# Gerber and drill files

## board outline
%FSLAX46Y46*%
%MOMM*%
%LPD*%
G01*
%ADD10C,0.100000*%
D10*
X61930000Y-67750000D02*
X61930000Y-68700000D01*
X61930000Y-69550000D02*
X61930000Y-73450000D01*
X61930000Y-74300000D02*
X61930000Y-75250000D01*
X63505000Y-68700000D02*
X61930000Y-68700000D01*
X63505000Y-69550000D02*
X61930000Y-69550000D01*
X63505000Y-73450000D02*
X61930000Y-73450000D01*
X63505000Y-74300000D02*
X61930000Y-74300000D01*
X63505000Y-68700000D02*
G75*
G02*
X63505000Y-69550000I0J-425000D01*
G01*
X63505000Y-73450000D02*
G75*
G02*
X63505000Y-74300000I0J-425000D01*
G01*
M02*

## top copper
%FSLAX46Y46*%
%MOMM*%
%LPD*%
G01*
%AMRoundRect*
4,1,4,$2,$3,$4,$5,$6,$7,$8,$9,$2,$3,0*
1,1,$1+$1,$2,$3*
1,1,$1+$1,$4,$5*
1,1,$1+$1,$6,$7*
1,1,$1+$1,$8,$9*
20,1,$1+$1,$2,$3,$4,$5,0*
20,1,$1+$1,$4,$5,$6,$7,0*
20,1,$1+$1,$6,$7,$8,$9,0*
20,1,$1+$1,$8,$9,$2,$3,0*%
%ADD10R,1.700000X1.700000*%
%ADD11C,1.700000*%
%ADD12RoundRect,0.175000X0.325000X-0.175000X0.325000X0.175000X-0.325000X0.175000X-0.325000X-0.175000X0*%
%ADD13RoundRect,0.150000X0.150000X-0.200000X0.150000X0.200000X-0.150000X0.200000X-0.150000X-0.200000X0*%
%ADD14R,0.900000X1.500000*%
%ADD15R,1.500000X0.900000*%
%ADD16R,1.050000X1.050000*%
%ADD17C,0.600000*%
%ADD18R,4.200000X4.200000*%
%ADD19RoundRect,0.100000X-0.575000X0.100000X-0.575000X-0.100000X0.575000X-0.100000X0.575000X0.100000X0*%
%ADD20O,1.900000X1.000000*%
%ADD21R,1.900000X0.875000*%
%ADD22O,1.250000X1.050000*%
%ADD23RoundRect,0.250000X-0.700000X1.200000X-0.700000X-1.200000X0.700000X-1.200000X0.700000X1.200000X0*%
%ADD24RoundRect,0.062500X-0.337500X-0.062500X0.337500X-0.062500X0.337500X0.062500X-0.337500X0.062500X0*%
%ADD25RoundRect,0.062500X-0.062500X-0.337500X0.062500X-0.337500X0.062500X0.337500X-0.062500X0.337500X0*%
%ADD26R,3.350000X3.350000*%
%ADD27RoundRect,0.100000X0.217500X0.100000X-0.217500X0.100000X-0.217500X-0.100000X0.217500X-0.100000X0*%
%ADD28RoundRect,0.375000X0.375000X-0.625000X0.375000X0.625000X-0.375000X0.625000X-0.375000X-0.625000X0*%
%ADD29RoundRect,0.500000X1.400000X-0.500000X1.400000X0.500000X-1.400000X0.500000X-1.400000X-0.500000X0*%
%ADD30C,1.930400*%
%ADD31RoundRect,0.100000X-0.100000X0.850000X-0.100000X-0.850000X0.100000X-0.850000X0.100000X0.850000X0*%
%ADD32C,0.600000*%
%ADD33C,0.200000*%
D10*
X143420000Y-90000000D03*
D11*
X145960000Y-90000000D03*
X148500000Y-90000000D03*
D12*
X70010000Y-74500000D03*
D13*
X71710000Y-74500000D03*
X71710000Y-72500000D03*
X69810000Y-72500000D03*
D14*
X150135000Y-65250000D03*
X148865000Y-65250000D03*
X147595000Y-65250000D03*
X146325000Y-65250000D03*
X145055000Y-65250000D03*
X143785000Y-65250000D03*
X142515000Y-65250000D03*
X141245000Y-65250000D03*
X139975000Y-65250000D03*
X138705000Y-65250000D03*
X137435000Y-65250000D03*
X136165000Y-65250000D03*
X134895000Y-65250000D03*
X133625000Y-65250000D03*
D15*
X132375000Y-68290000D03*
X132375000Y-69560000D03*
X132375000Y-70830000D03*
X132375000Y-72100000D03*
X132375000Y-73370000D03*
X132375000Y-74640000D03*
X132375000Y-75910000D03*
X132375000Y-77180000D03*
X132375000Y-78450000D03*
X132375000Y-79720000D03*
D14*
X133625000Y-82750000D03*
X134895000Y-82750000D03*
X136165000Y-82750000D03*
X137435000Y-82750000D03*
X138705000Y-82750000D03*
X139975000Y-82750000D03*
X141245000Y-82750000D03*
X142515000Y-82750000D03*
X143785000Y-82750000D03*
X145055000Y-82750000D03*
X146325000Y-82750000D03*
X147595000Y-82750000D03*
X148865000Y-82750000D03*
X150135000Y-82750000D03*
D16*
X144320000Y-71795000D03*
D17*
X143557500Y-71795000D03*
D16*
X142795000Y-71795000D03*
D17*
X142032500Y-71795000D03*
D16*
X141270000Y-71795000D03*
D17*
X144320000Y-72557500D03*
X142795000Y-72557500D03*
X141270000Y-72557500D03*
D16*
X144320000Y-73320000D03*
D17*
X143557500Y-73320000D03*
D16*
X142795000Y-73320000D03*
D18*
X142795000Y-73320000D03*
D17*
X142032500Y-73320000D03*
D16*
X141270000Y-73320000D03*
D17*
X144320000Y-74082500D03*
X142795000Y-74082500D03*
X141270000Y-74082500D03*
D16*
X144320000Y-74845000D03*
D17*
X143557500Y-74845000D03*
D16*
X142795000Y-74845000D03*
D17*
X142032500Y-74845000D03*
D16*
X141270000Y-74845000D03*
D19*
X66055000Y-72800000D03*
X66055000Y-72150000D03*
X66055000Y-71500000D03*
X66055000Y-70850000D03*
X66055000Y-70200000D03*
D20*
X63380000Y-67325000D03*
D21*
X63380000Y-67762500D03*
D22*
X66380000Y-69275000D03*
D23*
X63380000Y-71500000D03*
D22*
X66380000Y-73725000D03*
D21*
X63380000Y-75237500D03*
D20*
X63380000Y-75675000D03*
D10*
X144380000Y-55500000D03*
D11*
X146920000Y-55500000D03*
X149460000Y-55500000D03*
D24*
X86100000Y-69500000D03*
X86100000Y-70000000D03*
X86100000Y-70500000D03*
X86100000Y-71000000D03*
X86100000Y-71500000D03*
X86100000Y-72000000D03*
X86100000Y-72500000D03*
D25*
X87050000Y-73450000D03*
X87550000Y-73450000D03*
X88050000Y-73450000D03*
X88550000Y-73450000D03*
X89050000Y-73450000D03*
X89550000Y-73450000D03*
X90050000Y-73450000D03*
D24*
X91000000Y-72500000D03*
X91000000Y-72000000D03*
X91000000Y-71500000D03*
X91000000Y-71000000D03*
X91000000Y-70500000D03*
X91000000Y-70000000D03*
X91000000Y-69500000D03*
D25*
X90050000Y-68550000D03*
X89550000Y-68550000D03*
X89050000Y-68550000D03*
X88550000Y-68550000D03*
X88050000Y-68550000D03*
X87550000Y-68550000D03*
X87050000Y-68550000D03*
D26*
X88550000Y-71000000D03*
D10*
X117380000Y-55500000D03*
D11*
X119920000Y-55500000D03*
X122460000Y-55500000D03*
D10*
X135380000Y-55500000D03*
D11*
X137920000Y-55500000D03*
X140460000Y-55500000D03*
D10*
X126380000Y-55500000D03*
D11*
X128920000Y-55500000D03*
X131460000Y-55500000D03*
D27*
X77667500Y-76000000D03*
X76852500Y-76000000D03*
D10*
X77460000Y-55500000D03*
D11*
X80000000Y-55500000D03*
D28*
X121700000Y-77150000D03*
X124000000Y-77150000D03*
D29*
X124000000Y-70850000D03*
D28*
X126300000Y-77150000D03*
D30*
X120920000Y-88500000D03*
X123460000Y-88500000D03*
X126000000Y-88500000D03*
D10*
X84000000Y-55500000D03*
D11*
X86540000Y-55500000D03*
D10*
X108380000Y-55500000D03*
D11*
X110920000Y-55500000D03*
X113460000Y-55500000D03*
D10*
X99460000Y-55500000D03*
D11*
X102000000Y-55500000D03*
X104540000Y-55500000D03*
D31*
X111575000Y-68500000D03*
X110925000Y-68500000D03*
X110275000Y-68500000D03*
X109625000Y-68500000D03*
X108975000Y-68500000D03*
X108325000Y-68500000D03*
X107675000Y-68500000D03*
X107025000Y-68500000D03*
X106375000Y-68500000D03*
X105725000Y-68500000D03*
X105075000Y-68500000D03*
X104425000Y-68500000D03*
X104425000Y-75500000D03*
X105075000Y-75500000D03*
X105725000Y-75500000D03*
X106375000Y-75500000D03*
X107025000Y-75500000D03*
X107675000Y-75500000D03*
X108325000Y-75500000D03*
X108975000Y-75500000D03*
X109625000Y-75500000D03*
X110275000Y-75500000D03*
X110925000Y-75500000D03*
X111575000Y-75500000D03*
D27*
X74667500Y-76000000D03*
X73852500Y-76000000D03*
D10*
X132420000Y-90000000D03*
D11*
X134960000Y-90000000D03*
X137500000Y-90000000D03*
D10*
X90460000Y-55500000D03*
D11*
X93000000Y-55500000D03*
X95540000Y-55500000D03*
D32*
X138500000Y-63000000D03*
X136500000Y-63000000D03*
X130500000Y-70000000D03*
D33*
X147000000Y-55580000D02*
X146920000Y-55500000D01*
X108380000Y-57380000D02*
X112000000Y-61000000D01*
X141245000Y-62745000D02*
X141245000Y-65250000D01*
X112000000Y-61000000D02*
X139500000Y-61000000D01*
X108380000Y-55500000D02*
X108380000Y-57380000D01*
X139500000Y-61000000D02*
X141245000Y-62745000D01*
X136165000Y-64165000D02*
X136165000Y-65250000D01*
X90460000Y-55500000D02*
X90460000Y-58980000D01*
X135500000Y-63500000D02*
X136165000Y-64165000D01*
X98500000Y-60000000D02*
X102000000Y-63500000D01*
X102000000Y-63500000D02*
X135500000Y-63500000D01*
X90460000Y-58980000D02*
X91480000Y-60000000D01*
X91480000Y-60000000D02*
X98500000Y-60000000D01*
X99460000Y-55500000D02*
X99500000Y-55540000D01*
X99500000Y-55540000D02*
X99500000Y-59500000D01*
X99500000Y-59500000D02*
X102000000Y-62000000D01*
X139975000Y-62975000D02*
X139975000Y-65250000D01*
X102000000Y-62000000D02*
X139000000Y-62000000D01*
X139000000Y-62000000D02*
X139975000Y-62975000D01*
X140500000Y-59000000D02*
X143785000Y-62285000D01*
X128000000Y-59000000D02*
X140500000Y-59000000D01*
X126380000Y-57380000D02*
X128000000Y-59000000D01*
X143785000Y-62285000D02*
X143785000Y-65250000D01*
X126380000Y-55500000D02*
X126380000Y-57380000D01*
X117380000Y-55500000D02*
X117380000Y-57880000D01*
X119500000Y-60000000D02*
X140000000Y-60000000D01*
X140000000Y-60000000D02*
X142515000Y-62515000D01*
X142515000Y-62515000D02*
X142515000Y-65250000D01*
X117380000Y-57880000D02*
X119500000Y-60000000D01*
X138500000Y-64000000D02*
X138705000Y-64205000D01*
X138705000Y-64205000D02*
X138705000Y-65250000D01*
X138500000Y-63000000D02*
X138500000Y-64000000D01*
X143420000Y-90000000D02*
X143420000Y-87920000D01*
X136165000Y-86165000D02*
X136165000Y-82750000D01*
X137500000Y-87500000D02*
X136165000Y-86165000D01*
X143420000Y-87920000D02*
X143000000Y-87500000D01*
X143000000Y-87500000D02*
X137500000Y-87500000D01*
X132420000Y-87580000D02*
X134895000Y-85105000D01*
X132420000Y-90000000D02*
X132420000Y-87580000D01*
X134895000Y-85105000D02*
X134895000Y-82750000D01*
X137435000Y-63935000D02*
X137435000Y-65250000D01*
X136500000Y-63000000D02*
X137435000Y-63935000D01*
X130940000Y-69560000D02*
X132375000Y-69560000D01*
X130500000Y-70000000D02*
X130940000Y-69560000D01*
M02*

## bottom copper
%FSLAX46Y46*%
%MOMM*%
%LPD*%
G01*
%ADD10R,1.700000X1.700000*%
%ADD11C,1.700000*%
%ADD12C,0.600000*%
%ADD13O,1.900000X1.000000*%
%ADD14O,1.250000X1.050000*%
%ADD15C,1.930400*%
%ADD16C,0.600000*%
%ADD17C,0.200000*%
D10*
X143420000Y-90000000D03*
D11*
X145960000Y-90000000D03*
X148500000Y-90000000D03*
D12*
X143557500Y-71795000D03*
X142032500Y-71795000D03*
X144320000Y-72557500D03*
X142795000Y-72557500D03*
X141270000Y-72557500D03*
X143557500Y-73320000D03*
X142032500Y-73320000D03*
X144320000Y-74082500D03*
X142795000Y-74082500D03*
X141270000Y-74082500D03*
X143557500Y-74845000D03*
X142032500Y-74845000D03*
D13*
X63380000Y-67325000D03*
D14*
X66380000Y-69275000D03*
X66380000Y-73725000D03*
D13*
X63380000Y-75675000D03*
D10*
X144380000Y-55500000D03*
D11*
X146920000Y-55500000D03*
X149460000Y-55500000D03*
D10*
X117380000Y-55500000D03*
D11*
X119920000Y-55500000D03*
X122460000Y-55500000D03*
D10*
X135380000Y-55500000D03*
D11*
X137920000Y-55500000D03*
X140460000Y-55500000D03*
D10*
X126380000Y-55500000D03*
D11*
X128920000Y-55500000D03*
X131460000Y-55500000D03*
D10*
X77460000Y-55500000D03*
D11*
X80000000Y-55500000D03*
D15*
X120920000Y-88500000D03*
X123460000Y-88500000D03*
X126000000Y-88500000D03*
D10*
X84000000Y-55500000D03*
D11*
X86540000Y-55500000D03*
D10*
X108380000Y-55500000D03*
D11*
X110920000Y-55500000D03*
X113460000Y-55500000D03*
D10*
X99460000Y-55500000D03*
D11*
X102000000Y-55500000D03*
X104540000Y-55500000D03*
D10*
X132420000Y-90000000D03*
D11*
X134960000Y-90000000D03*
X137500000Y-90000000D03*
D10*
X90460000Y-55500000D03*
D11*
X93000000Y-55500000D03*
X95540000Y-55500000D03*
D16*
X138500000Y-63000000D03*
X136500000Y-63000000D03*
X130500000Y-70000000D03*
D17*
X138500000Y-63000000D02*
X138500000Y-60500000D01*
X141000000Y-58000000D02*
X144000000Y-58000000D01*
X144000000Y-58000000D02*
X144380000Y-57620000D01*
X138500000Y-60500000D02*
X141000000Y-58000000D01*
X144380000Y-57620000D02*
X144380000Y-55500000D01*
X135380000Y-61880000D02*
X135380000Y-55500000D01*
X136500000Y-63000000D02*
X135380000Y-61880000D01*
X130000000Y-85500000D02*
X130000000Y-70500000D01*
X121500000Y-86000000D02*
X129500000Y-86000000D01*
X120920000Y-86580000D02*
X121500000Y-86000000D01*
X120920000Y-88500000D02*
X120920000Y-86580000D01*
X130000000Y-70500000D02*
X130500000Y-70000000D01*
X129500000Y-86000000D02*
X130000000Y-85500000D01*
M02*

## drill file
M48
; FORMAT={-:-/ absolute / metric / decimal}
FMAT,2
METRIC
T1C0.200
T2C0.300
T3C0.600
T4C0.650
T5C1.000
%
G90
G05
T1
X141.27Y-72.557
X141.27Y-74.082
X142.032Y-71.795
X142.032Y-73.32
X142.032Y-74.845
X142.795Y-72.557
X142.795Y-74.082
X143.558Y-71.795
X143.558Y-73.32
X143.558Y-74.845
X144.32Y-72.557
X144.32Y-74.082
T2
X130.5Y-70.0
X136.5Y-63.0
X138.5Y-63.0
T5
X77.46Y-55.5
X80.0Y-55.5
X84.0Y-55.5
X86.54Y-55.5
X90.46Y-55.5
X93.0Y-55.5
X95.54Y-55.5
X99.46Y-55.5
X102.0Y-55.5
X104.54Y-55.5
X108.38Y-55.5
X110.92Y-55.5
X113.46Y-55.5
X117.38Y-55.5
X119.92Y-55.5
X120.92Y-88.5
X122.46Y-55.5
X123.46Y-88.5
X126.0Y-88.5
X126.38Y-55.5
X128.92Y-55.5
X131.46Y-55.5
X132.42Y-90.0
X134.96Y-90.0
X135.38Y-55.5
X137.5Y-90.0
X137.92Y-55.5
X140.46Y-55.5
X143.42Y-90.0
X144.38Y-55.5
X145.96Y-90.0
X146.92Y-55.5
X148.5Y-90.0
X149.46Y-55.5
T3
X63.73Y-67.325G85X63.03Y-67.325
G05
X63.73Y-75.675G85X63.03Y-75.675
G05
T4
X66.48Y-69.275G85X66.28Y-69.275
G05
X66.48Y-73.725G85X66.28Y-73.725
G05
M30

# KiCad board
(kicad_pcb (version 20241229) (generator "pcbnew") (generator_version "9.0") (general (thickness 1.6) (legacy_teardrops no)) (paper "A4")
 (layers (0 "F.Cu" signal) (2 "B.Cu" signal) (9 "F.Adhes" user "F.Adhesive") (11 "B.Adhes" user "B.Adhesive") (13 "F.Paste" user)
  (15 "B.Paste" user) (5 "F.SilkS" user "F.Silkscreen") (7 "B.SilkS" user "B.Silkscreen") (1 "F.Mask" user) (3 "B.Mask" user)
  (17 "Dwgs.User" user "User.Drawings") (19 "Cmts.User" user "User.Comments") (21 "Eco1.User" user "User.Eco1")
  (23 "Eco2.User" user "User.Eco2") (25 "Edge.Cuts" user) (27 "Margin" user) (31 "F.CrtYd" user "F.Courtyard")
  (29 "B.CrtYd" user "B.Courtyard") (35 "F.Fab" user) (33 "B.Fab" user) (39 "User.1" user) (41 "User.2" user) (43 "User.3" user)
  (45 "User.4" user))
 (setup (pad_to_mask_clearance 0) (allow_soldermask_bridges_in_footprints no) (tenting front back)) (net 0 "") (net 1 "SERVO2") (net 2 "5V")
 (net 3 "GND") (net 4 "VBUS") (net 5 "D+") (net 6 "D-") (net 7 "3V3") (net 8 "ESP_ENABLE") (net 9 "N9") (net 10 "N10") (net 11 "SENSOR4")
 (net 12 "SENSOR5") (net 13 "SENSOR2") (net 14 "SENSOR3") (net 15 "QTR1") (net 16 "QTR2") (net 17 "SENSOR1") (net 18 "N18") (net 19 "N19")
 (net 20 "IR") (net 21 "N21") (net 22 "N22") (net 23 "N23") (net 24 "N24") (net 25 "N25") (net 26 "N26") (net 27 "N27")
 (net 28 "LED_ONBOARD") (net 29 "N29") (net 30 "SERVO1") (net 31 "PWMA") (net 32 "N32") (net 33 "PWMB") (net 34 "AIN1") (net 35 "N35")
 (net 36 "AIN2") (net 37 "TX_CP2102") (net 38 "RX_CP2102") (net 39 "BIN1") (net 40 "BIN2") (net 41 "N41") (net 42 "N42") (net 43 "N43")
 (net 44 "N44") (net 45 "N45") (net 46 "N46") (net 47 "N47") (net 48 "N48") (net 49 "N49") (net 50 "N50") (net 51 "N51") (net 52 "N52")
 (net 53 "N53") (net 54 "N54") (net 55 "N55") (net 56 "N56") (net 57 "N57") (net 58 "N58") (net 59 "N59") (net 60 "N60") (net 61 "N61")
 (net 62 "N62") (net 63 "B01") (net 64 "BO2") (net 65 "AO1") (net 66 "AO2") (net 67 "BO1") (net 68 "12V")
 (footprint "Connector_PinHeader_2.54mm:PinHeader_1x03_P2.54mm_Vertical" (layer "F.Cu") (at 143.42 90 90)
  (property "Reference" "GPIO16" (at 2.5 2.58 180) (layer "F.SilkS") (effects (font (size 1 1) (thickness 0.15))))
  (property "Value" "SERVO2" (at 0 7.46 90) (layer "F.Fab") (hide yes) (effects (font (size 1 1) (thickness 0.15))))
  (pad "1" thru_hole rect (at 0 0 90) (size 1.7 1.7) (drill 1) (layers "*.Cu" "*.Mask") (remove_unused_layers no) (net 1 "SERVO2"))
  (pad "2" thru_hole circle (at 0 2.54 90) (size 1.7 1.7) (drill 1) (layers "*.Cu" "*.Mask") (remove_unused_layers no) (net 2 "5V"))
  (pad "3" thru_hole circle (at 0 5.08 90) (size 1.7 1.7) (drill 1) (layers "*.Cu" "*.Mask") (remove_unused_layers no) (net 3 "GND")))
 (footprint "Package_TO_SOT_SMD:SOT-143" (layer "F.Cu") (at 70.76 73.5 90)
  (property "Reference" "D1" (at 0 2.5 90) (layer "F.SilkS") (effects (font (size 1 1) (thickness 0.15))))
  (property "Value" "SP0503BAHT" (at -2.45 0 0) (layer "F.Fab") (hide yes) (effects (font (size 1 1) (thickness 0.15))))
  (pad "1" smd roundrect (at -1 -0.75 90) (size 0.7 1) (layers "F.Cu" "F.Mask" "F.Paste") (roundrect_rratio 0.25) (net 3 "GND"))
  (pad "2" smd roundrect (at -1 0.95 90) (size 0.7 0.6) (layers "F.Cu" "F.Mask" "F.Paste") (roundrect_rratio 0.25) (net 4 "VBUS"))
  (pad "3" smd roundrect (at 1 0.95 90) (size 0.7 0.6) (layers "F.Cu" "F.Mask" "F.Paste") (roundrect_rratio 0.25) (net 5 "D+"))
  (pad "4" smd roundrect (at 1 -0.95 90) (size 0.7 0.6) (layers "F.Cu" "F.Mask" "F.Paste") (roundrect_rratio 0.25) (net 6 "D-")))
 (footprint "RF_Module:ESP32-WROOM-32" (layer "F.Cu") (at 141.885 74 -90)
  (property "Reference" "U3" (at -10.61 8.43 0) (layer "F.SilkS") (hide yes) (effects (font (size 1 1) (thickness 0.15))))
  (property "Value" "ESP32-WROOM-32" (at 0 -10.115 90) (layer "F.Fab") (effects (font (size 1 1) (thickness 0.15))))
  (pad "1" smd rect (at -8.75 -8.25 270) (size 1.5 0.9) (layers "F.Cu" "F.Mask" "F.Paste") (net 3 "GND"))
  (pad "2" smd rect (at -8.75 -6.98 270) (size 1.5 0.9) (layers "F.Cu" "F.Mask" "F.Paste") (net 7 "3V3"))
  (pad "3" smd rect (at -8.75 -5.71 270) (size 1.5 0.9) (layers "F.Cu" "F.Mask" "F.Paste") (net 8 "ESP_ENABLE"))
  (pad "4" smd rect (at -8.75 -4.44 270) (size 1.5 0.9) (layers "F.Cu" "F.Mask" "F.Paste") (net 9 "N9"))
  (pad "5" smd rect (at -8.75 -3.17 270) (size 1.5 0.9) (layers "F.Cu" "F.Mask" "F.Paste") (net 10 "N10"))
  (pad "6" smd rect (at -8.75 -1.9 270) (size 1.5 0.9) (layers "F.Cu" "F.Mask" "F.Paste") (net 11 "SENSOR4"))
  (pad "7" smd rect (at -8.75 -0.63 270) (size 1.5 0.9) (layers "F.Cu" "F.Mask" "F.Paste") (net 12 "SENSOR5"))
  (pad "8" smd rect (at -8.75 0.64 270) (size 1.5 0.9) (layers "F.Cu" "F.Mask" "F.Paste") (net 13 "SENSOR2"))
  (pad "9" smd rect (at -8.75 1.91 270) (size 1.5 0.9) (layers "F.Cu" "F.Mask" "F.Paste") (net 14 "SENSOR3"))
  (pad "10" smd rect (at -8.75 3.18 270) (size 1.5 0.9) (layers "F.Cu" "F.Mask" "F.Paste") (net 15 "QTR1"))
  (pad "11" smd rect (at -8.75 4.45 270) (size 1.5 0.9) (layers "F.Cu" "F.Mask" "F.Paste") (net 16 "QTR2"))
  (pad "12" smd rect (at -8.75 5.72 270) (size 1.5 0.9) (layers "F.Cu" "F.Mask" "F.Paste") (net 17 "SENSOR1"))
  (pad "13" smd rect (at -8.75 6.99 270) (size 1.5 0.9) (layers "F.Cu" "F.Mask" "F.Paste") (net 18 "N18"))
  (pad "14" smd rect (at -8.75 8.26 270) (size 1.5 0.9) (layers "F.Cu" "F.Mask" "F.Paste") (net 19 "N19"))
  (pad "15" smd rect (at -5.71 9.51) (size 1.5 0.9) (layers "F.Cu" "F.Mask" "F.Paste") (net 3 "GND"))
  (pad "16" smd rect (at -4.44 9.51) (size 1.5 0.9) (layers "F.Cu" "F.Mask" "F.Paste") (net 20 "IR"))
  (pad "17" smd rect (at -3.17 9.51) (size 1.5 0.9) (layers "F.Cu" "F.Mask" "F.Paste") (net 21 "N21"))
  (pad "18" smd rect (at -1.9 9.51) (size 1.5 0.9) (layers "F.Cu" "F.Mask" "F.Paste") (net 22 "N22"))
  (pad "19" smd rect (at -0.63 9.51) (size 1.5 0.9) (layers "F.Cu" "F.Mask" "F.Paste") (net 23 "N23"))
  (pad "20" smd rect (at 0.64 9.51) (size 1.5 0.9) (layers "F.Cu" "F.Mask" "F.Paste") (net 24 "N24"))
  (pad "21" smd rect (at 1.91 9.51) (size 1.5 0.9) (layers "F.Cu" "F.Mask" "F.Paste") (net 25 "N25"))
  (pad "22" smd rect (at 3.18 9.51) (size 1.5 0.9) (layers "F.Cu" "F.Mask" "F.Paste") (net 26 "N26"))
  (pad "23" smd rect (at 4.45 9.51) (size 1.5 0.9) (layers "F.Cu" "F.Mask" "F.Paste") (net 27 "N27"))
  (pad "24" smd rect (at 5.72 9.51) (size 1.5 0.9) (layers "F.Cu" "F.Mask" "F.Paste") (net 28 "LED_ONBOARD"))
  (pad "25" smd rect (at 8.75 8.26 270) (size 1.5 0.9) (layers "F.Cu" "F.Mask" "F.Paste") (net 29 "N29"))
  (pad "26" smd rect (at 8.75 6.99 270) (size 1.5 0.9) (layers "F.Cu" "F.Mask" "F.Paste") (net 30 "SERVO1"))
  (pad "27" smd rect (at 8.75 5.72 270) (size 1.5 0.9) (layers "F.Cu" "F.Mask" "F.Paste") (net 1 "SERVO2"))
  (pad "28" smd rect (at 8.75 4.45 270) (size 1.5 0.9) (layers "F.Cu" "F.Mask" "F.Paste") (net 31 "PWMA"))
  (pad "29" smd rect (at 8.75 3.18 270) (size 1.5 0.9) (layers "F.Cu" "F.Mask" "F.Paste") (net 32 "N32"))
  (pad "30" smd rect (at 8.75 1.91 270) (size 1.5 0.9) (layers "F.Cu" "F.Mask" "F.Paste") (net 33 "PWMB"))
  (pad "31" smd rect (at 8.75 0.64 270) (size 1.5 0.9) (layers "F.Cu" "F.Mask" "F.Paste") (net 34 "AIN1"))
  (pad "32" smd rect (at 8.75 -0.63 270) (size 1.5 0.9) (layers "F.Cu" "F.Mask" "F.Paste") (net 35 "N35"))
  (pad "33" smd rect (at 8.75 -1.9 270) (size 1.5 0.9) (layers "F.Cu" "F.Mask" "F.Paste") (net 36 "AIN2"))
  (pad "34" smd rect (at 8.75 -3.17 270) (size 1.5 0.9) (layers "F.Cu" "F.Mask" "F.Paste") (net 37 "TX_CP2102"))
  (pad "35" smd rect (at 8.75 -4.44 270) (size 1.5 0.9) (layers "F.Cu" "F.Mask" "F.Paste") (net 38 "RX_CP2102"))
  (pad "36" smd rect (at 8.75 -5.71 270) (size 1.5 0.9) (layers "F.Cu" "F.Mask" "F.Paste") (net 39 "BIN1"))
  (pad "37" smd rect (at 8.75 -6.98 270) (size 1.5 0.9) (layers "F.Cu" "F.Mask" "F.Paste") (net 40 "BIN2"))
  (pad "38" smd rect (at 8.75 -8.25 270) (size 1.5 0.9) (layers "F.Cu" "F.Mask" "F.Paste") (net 3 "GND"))
  (pad "39" smd rect (at -2.205 -2.435 270) (size 1.05 1.05) (layers "F.Cu" "F.Paste") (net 3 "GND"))
  (pad "39" thru_hole circle (at -2.205 -1.6725 270) (size 0.6 0.6) (drill 0.2) (layers "*.Cu" "F.Mask") (remove_unused_layers no)
   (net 3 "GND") (zone_connect 2))
  (pad "39" smd rect (at -2.205 -0.91 270) (size 1.05 1.05) (layers "F.Cu" "F.Paste") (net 3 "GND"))
  (pad "39" thru_hole circle (at -2.205 -0.1475 270) (size 0.6 0.6) (drill 0.2) (layers "*.Cu" "F.Mask") (remove_unused_layers no)
   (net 3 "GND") (zone_connect 2))
  (pad "39" smd rect (at -2.205 0.615 270) (size 1.05 1.05) (layers "F.Cu" "F.Paste") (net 3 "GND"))
  (pad "39" thru_hole circle (at -1.4425 -2.435 270) (size 0.6 0.6) (drill 0.2) (layers "*.Cu" "F.Mask") (remove_unused_layers no)
   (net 3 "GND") (zone_connect 2))
  (pad "39" thru_hole circle (at -1.4425 -0.91 270) (size 0.6 0.6) (drill 0.2) (layers "*.Cu" "F.Mask") (remove_unused_layers no)
   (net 3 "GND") (zone_connect 2))
  (pad "39" thru_hole circle (at -1.4425 0.615 270) (size 0.6 0.6) (drill 0.2) (layers "*.Cu" "F.Mask") (remove_unused_layers no)
   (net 3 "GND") (zone_connect 2))
  (pad "39" smd rect (at -0.68 -2.435 270) (size 1.05 1.05) (layers "F.Cu" "F.Paste") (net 3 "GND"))
  (pad "39" thru_hole circle (at -0.68 -1.6725 270) (size 0.6 0.6) (drill 0.2) (layers "*.Cu" "F.Mask") (remove_unused_layers no)
   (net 3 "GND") (zone_connect 2))
  (pad "39" smd rect (at -0.68 -0.91 270) (size 1.05 1.05) (layers "F.Cu" "F.Paste") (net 3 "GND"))
  (pad "39" smd rect (at -0.68 -0.91 270) (size 4.2 4.2) (layers "F.Cu" "F.Mask") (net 3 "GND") (zone_connect 2))
  (pad "39" thru_hole circle (at -0.68 -0.1475 270) (size 0.6 0.6) (drill 0.2) (layers "*.Cu" "F.Mask") (remove_unused_layers no)
   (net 3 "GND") (zone_connect 2))
  (pad "39" smd rect (at -0.68 0.615 270) (size 1.05 1.05) (layers "F.Cu" "F.Paste") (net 3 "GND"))
  (pad "39" thru_hole circle (at 0.0825 -2.435 270) (size 0.6 0.6) (drill 0.2) (layers "*.Cu" "F.Mask") (remove_unused_layers no)
   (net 3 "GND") (zone_connect 2))
  (pad "39" thru_hole circle (at 0.0825 -0.91 270) (size 0.6 0.6) (drill 0.2) (layers "*.Cu" "F.Mask") (remove_unused_layers no)
   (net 3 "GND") (zone_connect 2))
  (pad "39" thru_hole circle (at 0.0825 0.615 270) (size 0.6 0.6) (drill 0.2) (layers "*.Cu" "F.Mask") (remove_unused_layers no)
   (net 3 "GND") (zone_connect 2))
  (pad "39" smd rect (at 0.845 -2.435 270) (size 1.05 1.05) (layers "F.Cu" "F.Paste") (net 3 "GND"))
  (pad "39" thru_hole circle (at 0.845 -1.6725 270) (size 0.6 0.6) (drill 0.2) (layers "*.Cu" "F.Mask") (remove_unused_layers no)
   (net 3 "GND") (zone_connect 2))
  (pad "39" smd rect (at 0.845 -0.91 270) (size 1.05 1.05) (layers "F.Cu" "F.Paste") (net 3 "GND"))
  (pad "39" thru_hole circle (at 0.845 -0.1475 270) (size 0.6 0.6) (drill 0.2) (layers "*.Cu" "F.Mask") (remove_unused_layers no)
   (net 3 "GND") (zone_connect 2))
  (pad "39" smd rect (at 0.845 0.615 270) (size 1.05 1.05) (layers "F.Cu" "F.Paste") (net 3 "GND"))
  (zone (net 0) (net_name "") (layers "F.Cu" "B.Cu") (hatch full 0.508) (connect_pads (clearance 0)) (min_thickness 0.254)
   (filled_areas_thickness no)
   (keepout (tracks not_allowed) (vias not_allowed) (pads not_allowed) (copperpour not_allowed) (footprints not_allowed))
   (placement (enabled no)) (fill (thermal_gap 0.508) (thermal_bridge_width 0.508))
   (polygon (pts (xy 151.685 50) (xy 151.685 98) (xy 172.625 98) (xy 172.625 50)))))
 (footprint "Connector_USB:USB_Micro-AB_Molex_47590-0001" (layer "F.Cu") (at 63.03 71.5 -90)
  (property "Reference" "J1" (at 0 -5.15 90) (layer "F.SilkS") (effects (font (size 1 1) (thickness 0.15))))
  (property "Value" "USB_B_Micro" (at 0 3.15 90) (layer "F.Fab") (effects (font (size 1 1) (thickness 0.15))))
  (fp_line (start -3.75 1.1) (end -2.8 1.1) (stroke (width 0.1) (type solid)) (layer "Edge.Cuts"))
  (fp_line (start -1.95 1.1) (end 1.95 1.1) (stroke (width 0.1) (type solid)) (layer "Edge.Cuts"))
  (fp_line (start 2.8 1.1) (end 3.75 1.1) (stroke (width 0.1) (type solid)) (layer "Edge.Cuts"))
  (fp_line (start -2.8 -0.475) (end -2.8 1.1) (stroke (width 0.1) (type solid)) (layer "Edge.Cuts"))
  (fp_line (start -1.95 -0.475) (end -1.95 1.1) (stroke (width 0.1) (type solid)) (layer "Edge.Cuts"))
  (fp_line (start 1.95 -0.475) (end 1.95 1.1) (stroke (width 0.1) (type solid)) (layer "Edge.Cuts"))
  (fp_line (start 2.8 -0.475) (end 2.8 1.1) (stroke (width 0.1) (type solid)) (layer "Edge.Cuts"))
  (fp_arc (start -2.8 -0.475) (mid -2.375 -0.9) (end -1.95 -0.475) (stroke (width 0.1) (type solid)) (layer "Edge.Cuts"))
  (fp_arc (start 1.95 -0.475) (mid 2.375 -0.9) (end 2.8 -0.475) (stroke (width 0.1) (type solid)) (layer "Edge.Cuts"))
  (pad "" smd rect (at -3.5 -0.35 270) (size 0.3 0.85) (layers "F.Paste"))
  (pad "" smd rect (at 3.5 -0.35 270) (size 0.3 0.85) (layers "F.Paste"))
  (pad "1" smd roundrect (at 1.3 -3.025 270) (size 0.4 1.35) (layers "F.Cu" "F.Mask" "F.Paste") (roundrect_rratio 0.25) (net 4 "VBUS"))
  (pad "2" smd roundrect (at 0.65 -3.025 270) (size 0.4 1.35) (layers "F.Cu" "F.Mask" "F.Paste") (roundrect_rratio 0.25) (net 6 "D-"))
  (pad "3" smd roundrect (at 0 -3.025 270) (size 0.4 1.35) (layers "F.Cu" "F.Mask" "F.Paste") (roundrect_rratio 0.25) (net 5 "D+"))
  (pad "4" smd roundrect (at -0.65 -3.025 270) (size 0.4 1.35) (layers "F.Cu" "F.Mask" "F.Paste") (roundrect_rratio 0.25) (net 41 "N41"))
  (pad "5" smd roundrect (at -1.3 -3.025 270) (size 0.4 1.35) (layers "F.Cu" "F.Mask" "F.Paste") (roundrect_rratio 0.25) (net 3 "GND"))
  (pad "6" thru_hole oval (at -4.175 -0.35 270) (size 1 1.9) (drill oval 0.6 1.3) (layers "*.Cu" "*.Mask") (remove_unused_layers no)
   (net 3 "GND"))
  (pad "6" smd rect (at -3.7375 -0.35 270) (size 0.875 1.9) (layers "F.Cu" "F.Mask") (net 3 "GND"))
  (pad "6" thru_hole oval (at -2.225 -3.35 270) (size 1.05 1.25) (drill oval 0.65 0.85) (layers "*.Cu" "*.Mask") (remove_unused_layers no)
   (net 3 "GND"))
  (pad "6" smd roundrect (at 0 -0.35 270) (size 2.9 1.9) (layers "F.Cu" "F.Mask" "F.Paste") (roundrect_rratio 0.1315789474) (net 3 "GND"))
  (pad "6" thru_hole oval (at 2.225 -3.35 270) (size 1.05 1.25) (drill oval 0.65 0.85) (layers "*.Cu" "*.Mask") (remove_unused_layers no)
   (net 3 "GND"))
  (pad "6" smd rect (at 3.7375 -0.35 270) (size 0.875 1.9) (layers "F.Cu" "F.Mask") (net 3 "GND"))
  (pad "6" thru_hole oval (at 4.175 -0.35 270) (size 1 1.9) (drill oval 0.6 1.3) (layers "*.Cu" "*.Mask") (remove_unused_layers no)
   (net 3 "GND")))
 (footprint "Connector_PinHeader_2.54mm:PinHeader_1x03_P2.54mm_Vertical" (layer "F.Cu") (at 144.38 55.5 90)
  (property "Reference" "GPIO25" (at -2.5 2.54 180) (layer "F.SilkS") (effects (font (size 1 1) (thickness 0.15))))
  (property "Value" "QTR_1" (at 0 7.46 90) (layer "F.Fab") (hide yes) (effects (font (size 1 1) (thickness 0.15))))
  (pad "1" thru_hole rect (at 0 0 90) (size 1.7 1.7) (drill 1) (layers "*.Cu" "*.Mask") (remove_unused_layers no) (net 15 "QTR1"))
  (pad "2" thru_hole circle (at 0 2.54 90) (size 1.7 1.7) (drill 1) (layers "*.Cu" "*.Mask") (remove_unused_layers no) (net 7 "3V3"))
  (pad "3" thru_hole circle (at 0 5.08 90) (size 1.7 1.7) (drill 1) (layers "*.Cu" "*.Mask") (remove_unused_layers no) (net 3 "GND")))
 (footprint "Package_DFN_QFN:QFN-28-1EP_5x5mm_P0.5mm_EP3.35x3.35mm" (layer "F.Cu") (at 88.55 71)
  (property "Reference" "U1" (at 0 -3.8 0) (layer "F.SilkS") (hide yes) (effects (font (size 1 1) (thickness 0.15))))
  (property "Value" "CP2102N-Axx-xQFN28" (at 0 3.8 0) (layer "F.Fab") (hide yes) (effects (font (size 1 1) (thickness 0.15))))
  (pad "" smd roundrect (at -1.12 -1.12) (size 0.9 0.9) (layers "F.Paste") (roundrect_rratio 0.25))
  (pad "" smd roundrect (at -1.12 0) (size 0.9 0.9) (layers "F.Paste") (roundrect_rratio 0.25))
  (pad "" smd roundrect (at -1.12 1.12) (size 0.9 0.9) (layers "F.Paste") (roundrect_rratio 0.25))
  (pad "" smd roundrect (at 0 -1.12) (size 0.9 0.9) (layers "F.Paste") (roundrect_rratio 0.25))
  (pad "" smd roundrect (at 0 0) (size 0.9 0.9) (layers "F.Paste") (roundrect_rratio 0.25))
  (pad "" smd roundrect (at 0 1.12) (size 0.9 0.9) (layers "F.Paste") (roundrect_rratio 0.25))
  (pad "" smd roundrect (at 1.12 -1.12) (size 0.9 0.9) (layers "F.Paste") (roundrect_rratio 0.25))
  (pad "" smd roundrect (at 1.12 0) (size 0.9 0.9) (layers "F.Paste") (roundrect_rratio 0.25))
  (pad "" smd roundrect (at 1.12 1.12) (size 0.9 0.9) (layers "F.Paste") (roundrect_rratio 0.25))
  (pad "1" smd roundrect (at -2.45 -1.5) (size 0.8 0.25) (layers "F.Cu" "F.Mask" "F.Paste") (roundrect_rratio 0.25) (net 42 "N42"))
  (pad "2" smd roundrect (at -2.45 -1) (size 0.8 0.25) (layers "F.Cu" "F.Mask" "F.Paste") (roundrect_rratio 0.25) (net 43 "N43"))
  (pad "3" smd roundrect (at -2.45 -0.5) (size 0.8 0.25) (layers "F.Cu" "F.Mask" "F.Paste") (roundrect_rratio 0.25) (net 3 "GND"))
  (pad "4" smd roundrect (at -2.45 0) (size 0.8 0.25) (layers "F.Cu" "F.Mask" "F.Paste") (roundrect_rratio 0.25) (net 5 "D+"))
  (pad "5" smd roundrect (at -2.45 0.5) (size 0.8 0.25) (layers "F.Cu" "F.Mask" "F.Paste") (roundrect_rratio 0.25) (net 6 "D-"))
  (pad "6" smd roundrect (at -2.45 1) (size 0.8 0.25) (layers "F.Cu" "F.Mask" "F.Paste") (roundrect_rratio 0.25) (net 7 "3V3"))
  (pad "7" smd roundrect (at -2.45 1.5) (size 0.8 0.25) (layers "F.Cu" "F.Mask" "F.Paste") (roundrect_rratio 0.25) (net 4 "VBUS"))
  (pad "8" smd roundrect (at -1.5 2.45) (size 0.25 0.8) (layers "F.Cu" "F.Mask" "F.Paste") (roundrect_rratio 0.25) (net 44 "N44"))
  (pad "9" smd roundrect (at -1 2.45) (size 0.25 0.8) (layers "F.Cu" "F.Mask" "F.Paste") (roundrect_rratio 0.25) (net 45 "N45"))
  (pad "10" smd roundrect (at -0.5 2.45) (size 0.25 0.8) (layers "F.Cu" "F.Mask" "F.Paste") (roundrect_rratio 0.25) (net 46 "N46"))
  (pad "11" smd roundrect (at 0 2.45) (size 0.25 0.8) (layers "F.Cu" "F.Mask" "F.Paste") (roundrect_rratio 0.25) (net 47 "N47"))
  (pad "12" smd roundrect (at 0.5 2.45) (size 0.25 0.8) (layers "F.Cu" "F.Mask" "F.Paste") (roundrect_rratio 0.25) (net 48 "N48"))
  (pad "13" smd roundrect (at 1 2.45) (size 0.25 0.8) (layers "F.Cu" "F.Mask" "F.Paste") (roundrect_rratio 0.25) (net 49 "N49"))
  (pad "14" smd roundrect (at 1.5 2.45) (size 0.25 0.8) (layers "F.Cu" "F.Mask" "F.Paste") (roundrect_rratio 0.25) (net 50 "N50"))
  (pad "15" smd roundrect (at 2.45 1.5) (size 0.8 0.25) (layers "F.Cu" "F.Mask" "F.Paste") (roundrect_rratio 0.25) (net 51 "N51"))
  (pad "16" smd roundrect (at 2.45 1) (size 0.8 0.25) (layers "F.Cu" "F.Mask" "F.Paste") (roundrect_rratio 0.25) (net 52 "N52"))
  (pad "17" smd roundrect (at 2.45 0.5) (size 0.8 0.25) (layers "F.Cu" "F.Mask" "F.Paste") (roundrect_rratio 0.25) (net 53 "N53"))
  (pad "18" smd roundrect (at 2.45 0) (size 0.8 0.25) (layers "F.Cu" "F.Mask" "F.Paste") (roundrect_rratio 0.25) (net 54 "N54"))
  (pad "19" smd roundrect (at 2.45 -0.5) (size 0.8 0.25) (layers "F.Cu" "F.Mask" "F.Paste") (roundrect_rratio 0.25) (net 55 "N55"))
  (pad "20" smd roundrect (at 2.45 -1) (size 0.8 0.25) (layers "F.Cu" "F.Mask" "F.Paste") (roundrect_rratio 0.25) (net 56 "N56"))
  (pad "21" smd roundrect (at 2.45 -1.5) (size 0.8 0.25) (layers "F.Cu" "F.Mask" "F.Paste") (roundrect_rratio 0.25) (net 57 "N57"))
  (pad "22" smd roundrect (at 1.5 -2.45) (size 0.25 0.8) (layers "F.Cu" "F.Mask" "F.Paste") (roundrect_rratio 0.25) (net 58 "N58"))
  (pad "23" smd roundrect (at 1 -2.45) (size 0.25 0.8) (layers "F.Cu" "F.Mask" "F.Paste") (roundrect_rratio 0.25) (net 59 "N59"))
  (pad "24" smd roundrect (at 0.5 -2.45) (size 0.25 0.8) (layers "F.Cu" "F.Mask" "F.Paste") (roundrect_rratio 0.25) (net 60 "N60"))
  (pad "25" smd roundrect (at 0 -2.45) (size 0.25 0.8) (layers "F.Cu" "F.Mask" "F.Paste") (roundrect_rratio 0.25) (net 38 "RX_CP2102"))
  (pad "26" smd roundrect (at -0.5 -2.45) (size 0.25 0.8) (layers "F.Cu" "F.Mask" "F.Paste") (roundrect_rratio 0.25) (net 37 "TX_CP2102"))
  (pad "27" smd roundrect (at -1 -2.45) (size 0.25 0.8) (layers "F.Cu" "F.Mask" "F.Paste") (roundrect_rratio 0.25) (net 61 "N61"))
  (pad "28" smd roundrect (at -1.5 -2.45) (size 0.25 0.8) (layers "F.Cu" "F.Mask" "F.Paste") (roundrect_rratio 0.25) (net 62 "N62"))
  (pad "29" smd rect (at 0 0) (size 3.35 3.35) (layers "F.Cu" "F.Mask") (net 3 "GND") (zone_connect 2)))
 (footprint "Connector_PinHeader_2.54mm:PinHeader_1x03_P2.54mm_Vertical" (layer "F.Cu") (at 117.38 55.5 90)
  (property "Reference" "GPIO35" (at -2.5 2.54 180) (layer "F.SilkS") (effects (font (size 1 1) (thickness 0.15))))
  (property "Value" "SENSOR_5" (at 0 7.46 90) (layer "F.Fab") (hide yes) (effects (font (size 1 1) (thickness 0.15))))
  (pad "1" thru_hole rect (at 0 0 90) (size 1.7 1.7) (drill 1) (layers "*.Cu" "*.Mask") (remove_unused_layers no) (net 12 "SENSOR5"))
  (pad "2" thru_hole circle (at 0 2.54 90) (size 1.7 1.7) (drill 1) (layers "*.Cu" "*.Mask") (remove_unused_layers no) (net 2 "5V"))
  (pad "3" thru_hole circle (at 0 5.08 90) (size 1.7 1.7) (drill 1) (layers "*.Cu" "*.Mask") (remove_unused_layers no) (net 3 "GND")))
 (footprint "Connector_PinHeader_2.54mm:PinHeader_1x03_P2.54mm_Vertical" (layer "F.Cu") (at 135.38 55.5 90)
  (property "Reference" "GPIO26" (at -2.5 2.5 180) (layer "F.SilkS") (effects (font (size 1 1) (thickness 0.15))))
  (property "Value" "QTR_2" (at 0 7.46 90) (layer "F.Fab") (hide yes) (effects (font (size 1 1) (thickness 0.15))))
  (pad "1" thru_hole rect (at 0 0 90) (size 1.7 1.7) (drill 1) (layers "*.Cu" "*.Mask") (remove_unused_layers no) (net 16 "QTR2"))
  (pad "2" thru_hole circle (at 0 2.54 90) (size 1.7 1.7) (drill 1) (layers "*.Cu" "*.Mask") (remove_unused_layers no) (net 7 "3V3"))
  (pad "3" thru_hole circle (at 0 5.08 90) (size 1.7 1.7) (drill 1) (layers "*.Cu" "*.Mask") (remove_unused_layers no) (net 3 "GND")))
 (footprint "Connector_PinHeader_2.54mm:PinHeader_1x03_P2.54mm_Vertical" (layer "F.Cu") (at 126.38 55.5 90)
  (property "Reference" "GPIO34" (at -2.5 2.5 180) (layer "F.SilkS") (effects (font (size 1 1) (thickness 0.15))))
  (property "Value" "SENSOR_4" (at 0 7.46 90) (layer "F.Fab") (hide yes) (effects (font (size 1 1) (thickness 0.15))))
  (pad "1" thru_hole rect (at 0 0 90) (size 1.7 1.7) (drill 1) (layers "*.Cu" "*.Mask") (remove_unused_layers no) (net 11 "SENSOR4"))
  (pad "2" thru_hole circle (at 0 2.54 90) (size 1.7 1.7) (drill 1) (layers "*.Cu" "*.Mask") (remove_unused_layers no) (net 2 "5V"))
  (pad "3" thru_hole circle (at 0 5.08 90) (size 1.7 1.7) (drill 1) (layers "*.Cu" "*.Mask") (remove_unused_layers no) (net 3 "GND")))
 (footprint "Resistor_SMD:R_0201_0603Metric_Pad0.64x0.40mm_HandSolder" (layer "F.Cu") (at 77.26 76 180)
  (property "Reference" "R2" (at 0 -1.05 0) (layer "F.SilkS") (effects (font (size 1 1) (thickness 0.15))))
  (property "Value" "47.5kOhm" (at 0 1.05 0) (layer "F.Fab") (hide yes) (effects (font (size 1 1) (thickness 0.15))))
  (pad "" smd roundrect (at -0.4325 0 180) (size 0.458 0.36) (layers "F.Paste") (roundrect_rratio 0.25))
  (pad "" smd roundrect (at 0.4325 0 180) (size 0.458 0.36) (layers "F.Paste") (roundrect_rratio 0.25))
  (pad "1" smd roundrect (at -0.4075 0 180) (size 0.635 0.4) (layers "F.Cu" "F.Mask") (roundrect_rratio 0.25) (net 3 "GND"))
  (pad "2" smd roundrect (at 0.4075 0 180) (size 0.635 0.4) (layers "F.Cu" "F.Mask") (roundrect_rratio 0.25) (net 44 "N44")))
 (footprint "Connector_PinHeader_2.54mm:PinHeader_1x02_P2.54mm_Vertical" (layer "F.Cu") (at 77.46 55.5 90)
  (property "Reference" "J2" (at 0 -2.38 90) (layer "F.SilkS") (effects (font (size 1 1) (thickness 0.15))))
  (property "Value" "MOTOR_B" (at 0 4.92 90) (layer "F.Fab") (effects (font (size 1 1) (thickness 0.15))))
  (pad "1" thru_hole rect (at 0 0 90) (size 1.7 1.7) (drill 1) (layers "*.Cu" "*.Mask") (remove_unused_layers no) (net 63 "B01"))
  (pad "2" thru_hole circle (at 0 2.54 90) (size 1.7 1.7) (drill 1) (layers "*.Cu" "*.Mask") (remove_unused_layers no) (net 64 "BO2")))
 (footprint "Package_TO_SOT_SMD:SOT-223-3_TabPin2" (layer "F.Cu") (at 124 74 90)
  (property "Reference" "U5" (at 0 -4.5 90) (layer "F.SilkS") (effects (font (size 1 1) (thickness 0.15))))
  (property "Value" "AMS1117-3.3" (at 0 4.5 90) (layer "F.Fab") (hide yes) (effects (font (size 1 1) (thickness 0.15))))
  (pad "1" smd roundrect (at -3.15 -2.3 90) (size 2 1.5) (layers "F.Cu" "F.Mask" "F.Paste") (roundrect_rratio 0.25) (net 3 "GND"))
  (pad "2" smd roundrect (at -3.15 0 90) (size 2 1.5) (layers "F.Cu" "F.Mask" "F.Paste") (roundrect_rratio 0.25) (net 7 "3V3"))
  (pad "2" smd roundrect (at 3.15 0 90) (size 2 3.8) (layers "F.Cu" "F.Mask" "F.Paste") (roundrect_rratio 0.25) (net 7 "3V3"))
  (pad "3" smd roundrect (at -3.15 2.3 90) (size 2 1.5) (layers "F.Cu" "F.Mask" "F.Paste") (roundrect_rratio 0.25) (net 2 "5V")))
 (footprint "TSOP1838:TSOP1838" (layer "F.Cu") (at 123.46 88.5)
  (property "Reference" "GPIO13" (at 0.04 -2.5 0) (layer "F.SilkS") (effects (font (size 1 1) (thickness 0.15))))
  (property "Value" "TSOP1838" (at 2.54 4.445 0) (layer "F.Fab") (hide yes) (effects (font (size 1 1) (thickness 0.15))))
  (pad "1" thru_hole circle (at -2.54 0) (size 1.9304 1.9304) (drill 1) (layers "*.Cu" "*.Mask") (remove_unused_layers no) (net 20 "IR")
   (solder_mask_margin 0.102))
  (pad "2" thru_hole circle (at 0 0) (size 1.9304 1.9304) (drill 1) (layers "*.Cu" "*.Mask") (remove_unused_layers no) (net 3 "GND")
   (solder_mask_margin 0.102))
  (pad "3" thru_hole circle (at 2.54 0) (size 1.9304 1.9304) (drill 1) (layers "*.Cu" "*.Mask") (remove_unused_layers no) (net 2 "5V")
   (solder_mask_margin 0.102)))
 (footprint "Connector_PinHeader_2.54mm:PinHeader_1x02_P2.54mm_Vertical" (layer "F.Cu") (at 84 55.5 90)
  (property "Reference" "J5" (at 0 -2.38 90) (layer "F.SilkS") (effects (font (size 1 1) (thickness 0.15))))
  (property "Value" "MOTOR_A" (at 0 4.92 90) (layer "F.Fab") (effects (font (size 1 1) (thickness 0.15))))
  (pad "1" thru_hole rect (at 0 0 90) (size 1.7 1.7) (drill 1) (layers "*.Cu" "*.Mask") (remove_unused_layers no) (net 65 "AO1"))
  (pad "2" thru_hole circle (at 0 2.54 90) (size 1.7 1.7) (drill 1) (layers "*.Cu" "*.Mask") (remove_unused_layers no) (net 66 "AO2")))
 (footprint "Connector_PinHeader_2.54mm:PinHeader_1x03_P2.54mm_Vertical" (layer "F.Cu") (at 108.38 55.5 90)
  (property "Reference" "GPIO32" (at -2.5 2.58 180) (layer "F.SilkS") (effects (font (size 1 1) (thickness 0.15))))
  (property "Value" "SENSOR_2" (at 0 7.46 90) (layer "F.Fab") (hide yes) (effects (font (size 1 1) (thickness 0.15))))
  (pad "1" thru_hole rect (at 0 0 90) (size 1.7 1.7) (drill 1) (layers "*.Cu" "*.Mask") (remove_unused_layers no) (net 13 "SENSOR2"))
  (pad "2" thru_hole circle (at 0 2.54 90) (size 1.7 1.7) (drill 1) (layers "*.Cu" "*.Mask") (remove_unused_layers no) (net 2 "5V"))
  (pad "3" thru_hole circle (at 0 5.08 90) (size 1.7 1.7) (drill 1) (layers "*.Cu" "*.Mask") (remove_unused_layers no) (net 3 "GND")))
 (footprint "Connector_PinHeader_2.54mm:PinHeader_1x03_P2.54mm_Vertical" (layer "F.Cu") (at 99.46 55.5 90)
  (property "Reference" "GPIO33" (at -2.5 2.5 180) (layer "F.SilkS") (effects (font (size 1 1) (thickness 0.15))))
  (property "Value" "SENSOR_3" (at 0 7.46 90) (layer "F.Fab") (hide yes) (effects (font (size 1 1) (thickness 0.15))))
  (pad "1" thru_hole rect (at 0 0 90) (size 1.7 1.7) (drill 1) (layers "*.Cu" "*.Mask") (remove_unused_layers no) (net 14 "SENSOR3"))
  (pad "2" thru_hole circle (at 0 2.54 90) (size 1.7 1.7) (drill 1) (layers "*.Cu" "*.Mask") (remove_unused_layers no) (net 2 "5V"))
  (pad "3" thru_hole circle (at 0 5.08 90) (size 1.7 1.7) (drill 1) (layers "*.Cu" "*.Mask") (remove_unused_layers no) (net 3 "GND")))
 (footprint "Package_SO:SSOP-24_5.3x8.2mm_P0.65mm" (layer "F.Cu") (at 108 72 -90)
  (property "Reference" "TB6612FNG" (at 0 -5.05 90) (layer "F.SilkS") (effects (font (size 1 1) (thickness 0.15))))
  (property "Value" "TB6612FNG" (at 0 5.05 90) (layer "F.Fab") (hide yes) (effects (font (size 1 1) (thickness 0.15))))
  (pad "1" smd roundrect (at -3.5 -3.575 270) (size 1.9 0.4) (layers "F.Cu" "F.Mask" "F.Paste") (roundrect_rratio 0.25) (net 65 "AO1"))
  (pad "2" smd roundrect (at -3.5 -2.925 270) (size 1.9 0.4) (layers "F.Cu" "F.Mask" "F.Paste") (roundrect_rratio 0.25) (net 65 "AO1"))
  (pad "3" smd roundrect (at -3.5 -2.275 270) (size 1.9 0.4) (layers "F.Cu" "F.Mask" "F.Paste") (roundrect_rratio 0.25) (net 3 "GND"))
  (pad "4" smd roundrect (at -3.5 -1.625 270) (size 1.9 0.4) (layers "F.Cu" "F.Mask" "F.Paste") (roundrect_rratio 0.25) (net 3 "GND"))
  (pad "5" smd roundrect (at -3.5 -0.975 270) (size 1.9 0.4) (layers "F.Cu" "F.Mask" "F.Paste") (roundrect_rratio 0.25) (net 66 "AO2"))
  (pad "6" smd roundrect (at -3.5 -0.325 270) (size 1.9 0.4) (layers "F.Cu" "F.Mask" "F.Paste") (roundrect_rratio 0.25) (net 66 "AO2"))
  (pad "7" smd roundrect (at -3.5 0.325 270) (size 1.9 0.4) (layers "F.Cu" "F.Mask" "F.Paste") (roundrect_rratio 0.25) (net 64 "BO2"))
  (pad "8" smd roundrect (at -3.5 0.975 270) (size 1.9 0.4) (layers "F.Cu" "F.Mask" "F.Paste") (roundrect_rratio 0.25) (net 64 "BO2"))
  (pad "9" smd roundrect (at -3.5 1.625 270) (size 1.9 0.4) (layers "F.Cu" "F.Mask" "F.Paste") (roundrect_rratio 0.25) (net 3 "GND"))
  (pad "10" smd roundrect (at -3.5 2.275 270) (size 1.9 0.4) (layers "F.Cu" "F.Mask" "F.Paste") (roundrect_rratio 0.25) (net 3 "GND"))
  (pad "11" smd roundrect (at -3.5 2.925 270) (size 1.9 0.4) (layers "F.Cu" "F.Mask" "F.Paste") (roundrect_rratio 0.25) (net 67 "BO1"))
  (pad "12" smd roundrect (at -3.5 3.575 270) (size 1.9 0.4) (layers "F.Cu" "F.Mask" "F.Paste") (roundrect_rratio 0.25) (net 67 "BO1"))
  (pad "13" smd roundrect (at 3.5 3.575 270) (size 1.9 0.4) (layers "F.Cu" "F.Mask" "F.Paste") (roundrect_rratio 0.25) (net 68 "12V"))
  (pad "14" smd roundrect (at 3.5 2.925 270) (size 1.9 0.4) (layers "F.Cu" "F.Mask" "F.Paste") (roundrect_rratio 0.25) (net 68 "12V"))
  (pad "15" smd roundrect (at 3.5 2.275 270) (size 1.9 0.4) (layers "F.Cu" "F.Mask" "F.Paste") (roundrect_rratio 0.25) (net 33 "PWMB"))
  (pad "16" smd roundrect (at 3.5 1.625 270) (size 1.9 0.4) (layers "F.Cu" "F.Mask" "F.Paste") (roundrect_rratio 0.25) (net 40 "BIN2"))
  (pad "17" smd roundrect (at 3.5 0.975 270) (size 1.9 0.4) (layers "F.Cu" "F.Mask" "F.Paste") (roundrect_rratio 0.25) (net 39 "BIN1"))
  (pad "18" smd roundrect (at 3.5 0.325 270) (size 1.9 0.4) (layers "F.Cu" "F.Mask" "F.Paste") (roundrect_rratio 0.25) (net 3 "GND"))
  (pad "19" smd roundrect (at 3.5 -0.325 270) (size 1.9 0.4) (layers "F.Cu" "F.Mask" "F.Paste") (roundrect_rratio 0.25) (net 2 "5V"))
  (pad "20" smd roundrect (at 3.5 -0.975 270) (size 1.9 0.4) (layers "F.Cu" "F.Mask" "F.Paste") (roundrect_rratio 0.25) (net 2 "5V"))
  (pad "21" smd roundrect (at 3.5 -1.625 270) (size 1.9 0.4) (layers "F.Cu" "F.Mask" "F.Paste") (roundrect_rratio 0.25) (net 34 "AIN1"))
  (pad "22" smd roundrect (at 3.5 -2.275 270) (size 1.9 0.4) (layers "F.Cu" "F.Mask" "F.Paste") (roundrect_rratio 0.25) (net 36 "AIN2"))
  (pad "23" smd roundrect (at 3.5 -2.925 270) (size 1.9 0.4) (layers "F.Cu" "F.Mask" "F.Paste") (roundrect_rratio 0.25) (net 31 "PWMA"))
  (pad "24" smd roundrect (at 3.5 -3.575 270) (size 1.9 0.4) (layers "F.Cu" "F.Mask" "F.Paste") (roundrect_rratio 0.25) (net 68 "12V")))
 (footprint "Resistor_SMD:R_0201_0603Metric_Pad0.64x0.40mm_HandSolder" (layer "F.Cu") (at 74.26 76 180)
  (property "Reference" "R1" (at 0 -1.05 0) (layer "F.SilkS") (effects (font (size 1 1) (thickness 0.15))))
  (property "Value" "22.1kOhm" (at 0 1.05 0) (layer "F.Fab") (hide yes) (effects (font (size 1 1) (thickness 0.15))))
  (pad "" smd roundrect (at -0.4325 0 180) (size 0.458 0.36) (layers "F.Paste") (roundrect_rratio 0.25))
  (pad "" smd roundrect (at 0.4325 0 180) (size 0.458 0.36) (layers "F.Paste") (roundrect_rratio 0.25))
  (pad "1" smd roundrect (at -0.4075 0 180) (size 0.635 0.4) (layers "F.Cu" "F.Mask") (roundrect_rratio 0.25) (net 44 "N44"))
  (pad "2" smd roundrect (at 0.4075 0 180) (size 0.635 0.4) (layers "F.Cu" "F.Mask") (roundrect_rratio 0.25) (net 4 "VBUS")))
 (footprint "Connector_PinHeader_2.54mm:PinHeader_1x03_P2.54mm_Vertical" (layer "F.Cu") (at 132.42 90 90)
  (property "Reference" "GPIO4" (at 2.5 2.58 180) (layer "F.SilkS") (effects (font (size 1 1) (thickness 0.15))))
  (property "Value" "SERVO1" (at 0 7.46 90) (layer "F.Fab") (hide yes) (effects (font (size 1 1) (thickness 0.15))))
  (pad "1" thru_hole rect (at 0 0 90) (size 1.7 1.7) (drill 1) (layers "*.Cu" "*.Mask") (remove_unused_layers no) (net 30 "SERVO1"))
  (pad "2" thru_hole circle (at 0 2.54 90) (size 1.7 1.7) (drill 1) (layers "*.Cu" "*.Mask") (remove_unused_layers no) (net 2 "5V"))
  (pad "3" thru_hole circle (at 0 5.08 90) (size 1.7 1.7) (drill 1) (layers "*.Cu" "*.Mask") (remove_unused_layers no) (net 3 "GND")))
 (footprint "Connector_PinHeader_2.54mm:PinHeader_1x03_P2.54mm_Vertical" (layer "F.Cu") (at 90.46 55.5 90)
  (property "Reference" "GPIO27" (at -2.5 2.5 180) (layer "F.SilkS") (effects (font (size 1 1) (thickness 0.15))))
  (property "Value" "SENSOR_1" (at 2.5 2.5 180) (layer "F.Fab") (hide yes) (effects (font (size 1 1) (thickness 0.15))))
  (pad "1" thru_hole rect (at 0 0 90) (size 1.7 1.7) (drill 1) (layers "*.Cu" "*.Mask") (remove_unused_layers no) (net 17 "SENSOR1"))
  (pad "2" thru_hole circle (at 0 2.54 90) (size 1.7 1.7) (drill 1) (layers "*.Cu" "*.Mask") (remove_unused_layers no) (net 2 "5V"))
  (pad "3" thru_hole circle (at 0 5.08 90) (size 1.7 1.7) (drill 1) (layers "*.Cu" "*.Mask") (remove_unused_layers no) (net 3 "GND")))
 (segment (start 147 55.58) (end 146.92 55.5) (width 0.2) (layer "F.Cu") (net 7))
 (segment (start 108.38 57.38) (end 112 61) (width 0.2) (layer "F.Cu") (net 13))
 (segment (start 141.245 62.745) (end 141.245 65.25) (width 0.2) (layer "F.Cu") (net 13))
 (segment (start 112 61) (end 139.5 61) (width 0.2) (layer "F.Cu") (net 13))
 (segment (start 108.38 55.5) (end 108.38 57.38) (width 0.2) (layer "F.Cu") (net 13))
 (segment (start 139.5 61) (end 141.245 62.745) (width 0.2) (layer "F.Cu") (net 13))
 (segment (start 136.165 64.165) (end 136.165 65.25) (width 0.2) (layer "F.Cu") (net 17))
 (segment (start 90.46 55.5) (end 90.46 58.98) (width 0.2) (layer "F.Cu") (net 17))
 (segment (start 135.5 63.5) (end 136.165 64.165) (width 0.2) (layer "F.Cu") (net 17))
 (segment (start 98.5 60) (end 102 63.5) (width 0.2) (layer "F.Cu") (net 17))
 (segment (start 102 63.5) (end 135.5 63.5) (width 0.2) (layer "F.Cu") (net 17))
 (segment (start 90.46 58.98) (end 91.48 60) (width 0.2) (layer "F.Cu") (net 17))
 (segment (start 91.48 60) (end 98.5 60) (width 0.2) (layer "F.Cu") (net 17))
 (segment (start 99.46 55.5) (end 99.5 55.54) (width 0.2) (layer "F.Cu") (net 14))
 (segment (start 99.5 55.54) (end 99.5 59.5) (width 0.2) (layer "F.Cu") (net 14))
 (segment (start 99.5 59.5) (end 102 62) (width 0.2) (layer "F.Cu") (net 14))
 (segment (start 139.975 62.975) (end 139.975 65.25) (width 0.2) (layer "F.Cu") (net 14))
 (segment (start 102 62) (end 139 62) (width 0.2) (layer "F.Cu") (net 14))
 (segment (start 139 62) (end 139.975 62.975) (width 0.2) (layer "F.Cu") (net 14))
 (segment (start 140.5 59) (end 143.785 62.285) (width 0.2) (layer "F.Cu") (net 11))
 (segment (start 128 59) (end 140.5 59) (width 0.2) (layer "F.Cu") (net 11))
 (segment (start 126.38 57.38) (end 128 59) (width 0.2) (layer "F.Cu") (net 11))
 (segment (start 143.785 62.285) (end 143.785 65.25) (width 0.2) (layer "F.Cu") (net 11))
 (segment (start 126.38 55.5) (end 126.38 57.38) (width 0.2) (layer "F.Cu") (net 11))
 (segment (start 117.38 55.5) (end 117.38 57.88) (width 0.2) (layer "F.Cu") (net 12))
 (segment (start 119.5 60) (end 140 60) (width 0.2) (layer "F.Cu") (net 12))
 (segment (start 140 60) (end 142.515 62.515) (width 0.2) (layer "F.Cu") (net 12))
 (segment (start 142.515 62.515) (end 142.515 65.25) (width 0.2) (layer "F.Cu") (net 12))
 (segment (start 117.38 57.88) (end 119.5 60) (width 0.2) (layer "F.Cu") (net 12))
 (segment (start 138.5 64) (end 138.705 64.205) (width 0.2) (layer "F.Cu") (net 15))
 (segment (start 138.705 64.205) (end 138.705 65.25) (width 0.2) (layer "F.Cu") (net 15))
 (segment (start 138.5 63) (end 138.5 64) (width 0.2) (layer "F.Cu") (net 15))
 (via (at 138.5 63) (size 0.6) (drill 0.3) (layers "F.Cu" "B.Cu") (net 15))
 (segment (start 138.5 63) (end 138.5 60.5) (width 0.2) (layer "B.Cu") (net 15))
 (segment (start 141 58) (end 144 58) (width 0.2) (layer "B.Cu") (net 15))
 (segment (start 144 58) (end 144.38 57.62) (width 0.2) (layer "B.Cu") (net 15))
 (segment (start 138.5 60.5) (end 141 58) (width 0.2) (layer "B.Cu") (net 15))
 (segment (start 144.38 57.62) (end 144.38 55.5) (width 0.2) (layer "B.Cu") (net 15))
 (segment (start 143.42 90) (end 143.42 87.92) (width 0.2) (layer "F.Cu") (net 1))
 (segment (start 136.165 86.165) (end 136.165 82.75) (width 0.2) (layer "F.Cu") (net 1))
 (segment (start 137.5 87.5) (end 136.165 86.165) (width 0.2) (layer "F.Cu") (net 1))
 (segment (start 143.42 87.92) (end 143 87.5) (width 0.2) (layer "F.Cu") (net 1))
 (segment (start 143 87.5) (end 137.5 87.5) (width 0.2) (layer "F.Cu") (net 1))
 (segment (start 132.42 87.58) (end 134.895 85.105) (width 0.2) (layer "F.Cu") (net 30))
 (segment (start 132.42 90) (end 132.42 87.58) (width 0.2) (layer "F.Cu") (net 30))
 (segment (start 134.895 85.105) (end 134.895 82.75) (width 0.2) (layer "F.Cu") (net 30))
 (segment (start 137.435 63.935) (end 137.435 65.25) (width 0.2) (layer "F.Cu") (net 16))
 (segment (start 136.5 63) (end 137.435 63.935) (width 0.2) (layer "F.Cu") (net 16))
 (via (at 136.5 63) (size 0.6) (drill 0.3) (layers "F.Cu" "B.Cu") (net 16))
 (segment (start 135.38 61.88) (end 135.38 55.5) (width 0.2) (layer "B.Cu") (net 16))
 (segment (start 136.5 63) (end 135.38 61.88) (width 0.2) (layer "B.Cu") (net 16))
 (segment (start 130.94 69.56) (end 132.375 69.56) (width 0.2) (layer "F.Cu") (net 20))
 (segment (start 130.5 70) (end 130.94 69.56) (width 0.2) (layer "F.Cu") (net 20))
 (via (at 130.5 70) (size 0.6) (drill 0.3) (layers "F.Cu" "B.Cu") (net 20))
 (segment (start 130 85.5) (end 130 70.5) (width 0.2) (layer "B.Cu") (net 20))
 (segment (start 121.5 86) (end 129.5 86) (width 0.2) (layer "B.Cu") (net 20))
 (segment (start 120.92 86.58) (end 121.5 86) (width 0.2) (layer "B.Cu") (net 20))
 (segment (start 120.92 88.5) (end 120.92 86.58) (width 0.2) (layer "B.Cu") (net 20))
 (segment (start 130 70.5) (end 130.5 70) (width 0.2) (layer "B.Cu") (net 20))
 (segment (start 129.5 86) (end 130 85.5) (width 0.2) (layer "B.Cu") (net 20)))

